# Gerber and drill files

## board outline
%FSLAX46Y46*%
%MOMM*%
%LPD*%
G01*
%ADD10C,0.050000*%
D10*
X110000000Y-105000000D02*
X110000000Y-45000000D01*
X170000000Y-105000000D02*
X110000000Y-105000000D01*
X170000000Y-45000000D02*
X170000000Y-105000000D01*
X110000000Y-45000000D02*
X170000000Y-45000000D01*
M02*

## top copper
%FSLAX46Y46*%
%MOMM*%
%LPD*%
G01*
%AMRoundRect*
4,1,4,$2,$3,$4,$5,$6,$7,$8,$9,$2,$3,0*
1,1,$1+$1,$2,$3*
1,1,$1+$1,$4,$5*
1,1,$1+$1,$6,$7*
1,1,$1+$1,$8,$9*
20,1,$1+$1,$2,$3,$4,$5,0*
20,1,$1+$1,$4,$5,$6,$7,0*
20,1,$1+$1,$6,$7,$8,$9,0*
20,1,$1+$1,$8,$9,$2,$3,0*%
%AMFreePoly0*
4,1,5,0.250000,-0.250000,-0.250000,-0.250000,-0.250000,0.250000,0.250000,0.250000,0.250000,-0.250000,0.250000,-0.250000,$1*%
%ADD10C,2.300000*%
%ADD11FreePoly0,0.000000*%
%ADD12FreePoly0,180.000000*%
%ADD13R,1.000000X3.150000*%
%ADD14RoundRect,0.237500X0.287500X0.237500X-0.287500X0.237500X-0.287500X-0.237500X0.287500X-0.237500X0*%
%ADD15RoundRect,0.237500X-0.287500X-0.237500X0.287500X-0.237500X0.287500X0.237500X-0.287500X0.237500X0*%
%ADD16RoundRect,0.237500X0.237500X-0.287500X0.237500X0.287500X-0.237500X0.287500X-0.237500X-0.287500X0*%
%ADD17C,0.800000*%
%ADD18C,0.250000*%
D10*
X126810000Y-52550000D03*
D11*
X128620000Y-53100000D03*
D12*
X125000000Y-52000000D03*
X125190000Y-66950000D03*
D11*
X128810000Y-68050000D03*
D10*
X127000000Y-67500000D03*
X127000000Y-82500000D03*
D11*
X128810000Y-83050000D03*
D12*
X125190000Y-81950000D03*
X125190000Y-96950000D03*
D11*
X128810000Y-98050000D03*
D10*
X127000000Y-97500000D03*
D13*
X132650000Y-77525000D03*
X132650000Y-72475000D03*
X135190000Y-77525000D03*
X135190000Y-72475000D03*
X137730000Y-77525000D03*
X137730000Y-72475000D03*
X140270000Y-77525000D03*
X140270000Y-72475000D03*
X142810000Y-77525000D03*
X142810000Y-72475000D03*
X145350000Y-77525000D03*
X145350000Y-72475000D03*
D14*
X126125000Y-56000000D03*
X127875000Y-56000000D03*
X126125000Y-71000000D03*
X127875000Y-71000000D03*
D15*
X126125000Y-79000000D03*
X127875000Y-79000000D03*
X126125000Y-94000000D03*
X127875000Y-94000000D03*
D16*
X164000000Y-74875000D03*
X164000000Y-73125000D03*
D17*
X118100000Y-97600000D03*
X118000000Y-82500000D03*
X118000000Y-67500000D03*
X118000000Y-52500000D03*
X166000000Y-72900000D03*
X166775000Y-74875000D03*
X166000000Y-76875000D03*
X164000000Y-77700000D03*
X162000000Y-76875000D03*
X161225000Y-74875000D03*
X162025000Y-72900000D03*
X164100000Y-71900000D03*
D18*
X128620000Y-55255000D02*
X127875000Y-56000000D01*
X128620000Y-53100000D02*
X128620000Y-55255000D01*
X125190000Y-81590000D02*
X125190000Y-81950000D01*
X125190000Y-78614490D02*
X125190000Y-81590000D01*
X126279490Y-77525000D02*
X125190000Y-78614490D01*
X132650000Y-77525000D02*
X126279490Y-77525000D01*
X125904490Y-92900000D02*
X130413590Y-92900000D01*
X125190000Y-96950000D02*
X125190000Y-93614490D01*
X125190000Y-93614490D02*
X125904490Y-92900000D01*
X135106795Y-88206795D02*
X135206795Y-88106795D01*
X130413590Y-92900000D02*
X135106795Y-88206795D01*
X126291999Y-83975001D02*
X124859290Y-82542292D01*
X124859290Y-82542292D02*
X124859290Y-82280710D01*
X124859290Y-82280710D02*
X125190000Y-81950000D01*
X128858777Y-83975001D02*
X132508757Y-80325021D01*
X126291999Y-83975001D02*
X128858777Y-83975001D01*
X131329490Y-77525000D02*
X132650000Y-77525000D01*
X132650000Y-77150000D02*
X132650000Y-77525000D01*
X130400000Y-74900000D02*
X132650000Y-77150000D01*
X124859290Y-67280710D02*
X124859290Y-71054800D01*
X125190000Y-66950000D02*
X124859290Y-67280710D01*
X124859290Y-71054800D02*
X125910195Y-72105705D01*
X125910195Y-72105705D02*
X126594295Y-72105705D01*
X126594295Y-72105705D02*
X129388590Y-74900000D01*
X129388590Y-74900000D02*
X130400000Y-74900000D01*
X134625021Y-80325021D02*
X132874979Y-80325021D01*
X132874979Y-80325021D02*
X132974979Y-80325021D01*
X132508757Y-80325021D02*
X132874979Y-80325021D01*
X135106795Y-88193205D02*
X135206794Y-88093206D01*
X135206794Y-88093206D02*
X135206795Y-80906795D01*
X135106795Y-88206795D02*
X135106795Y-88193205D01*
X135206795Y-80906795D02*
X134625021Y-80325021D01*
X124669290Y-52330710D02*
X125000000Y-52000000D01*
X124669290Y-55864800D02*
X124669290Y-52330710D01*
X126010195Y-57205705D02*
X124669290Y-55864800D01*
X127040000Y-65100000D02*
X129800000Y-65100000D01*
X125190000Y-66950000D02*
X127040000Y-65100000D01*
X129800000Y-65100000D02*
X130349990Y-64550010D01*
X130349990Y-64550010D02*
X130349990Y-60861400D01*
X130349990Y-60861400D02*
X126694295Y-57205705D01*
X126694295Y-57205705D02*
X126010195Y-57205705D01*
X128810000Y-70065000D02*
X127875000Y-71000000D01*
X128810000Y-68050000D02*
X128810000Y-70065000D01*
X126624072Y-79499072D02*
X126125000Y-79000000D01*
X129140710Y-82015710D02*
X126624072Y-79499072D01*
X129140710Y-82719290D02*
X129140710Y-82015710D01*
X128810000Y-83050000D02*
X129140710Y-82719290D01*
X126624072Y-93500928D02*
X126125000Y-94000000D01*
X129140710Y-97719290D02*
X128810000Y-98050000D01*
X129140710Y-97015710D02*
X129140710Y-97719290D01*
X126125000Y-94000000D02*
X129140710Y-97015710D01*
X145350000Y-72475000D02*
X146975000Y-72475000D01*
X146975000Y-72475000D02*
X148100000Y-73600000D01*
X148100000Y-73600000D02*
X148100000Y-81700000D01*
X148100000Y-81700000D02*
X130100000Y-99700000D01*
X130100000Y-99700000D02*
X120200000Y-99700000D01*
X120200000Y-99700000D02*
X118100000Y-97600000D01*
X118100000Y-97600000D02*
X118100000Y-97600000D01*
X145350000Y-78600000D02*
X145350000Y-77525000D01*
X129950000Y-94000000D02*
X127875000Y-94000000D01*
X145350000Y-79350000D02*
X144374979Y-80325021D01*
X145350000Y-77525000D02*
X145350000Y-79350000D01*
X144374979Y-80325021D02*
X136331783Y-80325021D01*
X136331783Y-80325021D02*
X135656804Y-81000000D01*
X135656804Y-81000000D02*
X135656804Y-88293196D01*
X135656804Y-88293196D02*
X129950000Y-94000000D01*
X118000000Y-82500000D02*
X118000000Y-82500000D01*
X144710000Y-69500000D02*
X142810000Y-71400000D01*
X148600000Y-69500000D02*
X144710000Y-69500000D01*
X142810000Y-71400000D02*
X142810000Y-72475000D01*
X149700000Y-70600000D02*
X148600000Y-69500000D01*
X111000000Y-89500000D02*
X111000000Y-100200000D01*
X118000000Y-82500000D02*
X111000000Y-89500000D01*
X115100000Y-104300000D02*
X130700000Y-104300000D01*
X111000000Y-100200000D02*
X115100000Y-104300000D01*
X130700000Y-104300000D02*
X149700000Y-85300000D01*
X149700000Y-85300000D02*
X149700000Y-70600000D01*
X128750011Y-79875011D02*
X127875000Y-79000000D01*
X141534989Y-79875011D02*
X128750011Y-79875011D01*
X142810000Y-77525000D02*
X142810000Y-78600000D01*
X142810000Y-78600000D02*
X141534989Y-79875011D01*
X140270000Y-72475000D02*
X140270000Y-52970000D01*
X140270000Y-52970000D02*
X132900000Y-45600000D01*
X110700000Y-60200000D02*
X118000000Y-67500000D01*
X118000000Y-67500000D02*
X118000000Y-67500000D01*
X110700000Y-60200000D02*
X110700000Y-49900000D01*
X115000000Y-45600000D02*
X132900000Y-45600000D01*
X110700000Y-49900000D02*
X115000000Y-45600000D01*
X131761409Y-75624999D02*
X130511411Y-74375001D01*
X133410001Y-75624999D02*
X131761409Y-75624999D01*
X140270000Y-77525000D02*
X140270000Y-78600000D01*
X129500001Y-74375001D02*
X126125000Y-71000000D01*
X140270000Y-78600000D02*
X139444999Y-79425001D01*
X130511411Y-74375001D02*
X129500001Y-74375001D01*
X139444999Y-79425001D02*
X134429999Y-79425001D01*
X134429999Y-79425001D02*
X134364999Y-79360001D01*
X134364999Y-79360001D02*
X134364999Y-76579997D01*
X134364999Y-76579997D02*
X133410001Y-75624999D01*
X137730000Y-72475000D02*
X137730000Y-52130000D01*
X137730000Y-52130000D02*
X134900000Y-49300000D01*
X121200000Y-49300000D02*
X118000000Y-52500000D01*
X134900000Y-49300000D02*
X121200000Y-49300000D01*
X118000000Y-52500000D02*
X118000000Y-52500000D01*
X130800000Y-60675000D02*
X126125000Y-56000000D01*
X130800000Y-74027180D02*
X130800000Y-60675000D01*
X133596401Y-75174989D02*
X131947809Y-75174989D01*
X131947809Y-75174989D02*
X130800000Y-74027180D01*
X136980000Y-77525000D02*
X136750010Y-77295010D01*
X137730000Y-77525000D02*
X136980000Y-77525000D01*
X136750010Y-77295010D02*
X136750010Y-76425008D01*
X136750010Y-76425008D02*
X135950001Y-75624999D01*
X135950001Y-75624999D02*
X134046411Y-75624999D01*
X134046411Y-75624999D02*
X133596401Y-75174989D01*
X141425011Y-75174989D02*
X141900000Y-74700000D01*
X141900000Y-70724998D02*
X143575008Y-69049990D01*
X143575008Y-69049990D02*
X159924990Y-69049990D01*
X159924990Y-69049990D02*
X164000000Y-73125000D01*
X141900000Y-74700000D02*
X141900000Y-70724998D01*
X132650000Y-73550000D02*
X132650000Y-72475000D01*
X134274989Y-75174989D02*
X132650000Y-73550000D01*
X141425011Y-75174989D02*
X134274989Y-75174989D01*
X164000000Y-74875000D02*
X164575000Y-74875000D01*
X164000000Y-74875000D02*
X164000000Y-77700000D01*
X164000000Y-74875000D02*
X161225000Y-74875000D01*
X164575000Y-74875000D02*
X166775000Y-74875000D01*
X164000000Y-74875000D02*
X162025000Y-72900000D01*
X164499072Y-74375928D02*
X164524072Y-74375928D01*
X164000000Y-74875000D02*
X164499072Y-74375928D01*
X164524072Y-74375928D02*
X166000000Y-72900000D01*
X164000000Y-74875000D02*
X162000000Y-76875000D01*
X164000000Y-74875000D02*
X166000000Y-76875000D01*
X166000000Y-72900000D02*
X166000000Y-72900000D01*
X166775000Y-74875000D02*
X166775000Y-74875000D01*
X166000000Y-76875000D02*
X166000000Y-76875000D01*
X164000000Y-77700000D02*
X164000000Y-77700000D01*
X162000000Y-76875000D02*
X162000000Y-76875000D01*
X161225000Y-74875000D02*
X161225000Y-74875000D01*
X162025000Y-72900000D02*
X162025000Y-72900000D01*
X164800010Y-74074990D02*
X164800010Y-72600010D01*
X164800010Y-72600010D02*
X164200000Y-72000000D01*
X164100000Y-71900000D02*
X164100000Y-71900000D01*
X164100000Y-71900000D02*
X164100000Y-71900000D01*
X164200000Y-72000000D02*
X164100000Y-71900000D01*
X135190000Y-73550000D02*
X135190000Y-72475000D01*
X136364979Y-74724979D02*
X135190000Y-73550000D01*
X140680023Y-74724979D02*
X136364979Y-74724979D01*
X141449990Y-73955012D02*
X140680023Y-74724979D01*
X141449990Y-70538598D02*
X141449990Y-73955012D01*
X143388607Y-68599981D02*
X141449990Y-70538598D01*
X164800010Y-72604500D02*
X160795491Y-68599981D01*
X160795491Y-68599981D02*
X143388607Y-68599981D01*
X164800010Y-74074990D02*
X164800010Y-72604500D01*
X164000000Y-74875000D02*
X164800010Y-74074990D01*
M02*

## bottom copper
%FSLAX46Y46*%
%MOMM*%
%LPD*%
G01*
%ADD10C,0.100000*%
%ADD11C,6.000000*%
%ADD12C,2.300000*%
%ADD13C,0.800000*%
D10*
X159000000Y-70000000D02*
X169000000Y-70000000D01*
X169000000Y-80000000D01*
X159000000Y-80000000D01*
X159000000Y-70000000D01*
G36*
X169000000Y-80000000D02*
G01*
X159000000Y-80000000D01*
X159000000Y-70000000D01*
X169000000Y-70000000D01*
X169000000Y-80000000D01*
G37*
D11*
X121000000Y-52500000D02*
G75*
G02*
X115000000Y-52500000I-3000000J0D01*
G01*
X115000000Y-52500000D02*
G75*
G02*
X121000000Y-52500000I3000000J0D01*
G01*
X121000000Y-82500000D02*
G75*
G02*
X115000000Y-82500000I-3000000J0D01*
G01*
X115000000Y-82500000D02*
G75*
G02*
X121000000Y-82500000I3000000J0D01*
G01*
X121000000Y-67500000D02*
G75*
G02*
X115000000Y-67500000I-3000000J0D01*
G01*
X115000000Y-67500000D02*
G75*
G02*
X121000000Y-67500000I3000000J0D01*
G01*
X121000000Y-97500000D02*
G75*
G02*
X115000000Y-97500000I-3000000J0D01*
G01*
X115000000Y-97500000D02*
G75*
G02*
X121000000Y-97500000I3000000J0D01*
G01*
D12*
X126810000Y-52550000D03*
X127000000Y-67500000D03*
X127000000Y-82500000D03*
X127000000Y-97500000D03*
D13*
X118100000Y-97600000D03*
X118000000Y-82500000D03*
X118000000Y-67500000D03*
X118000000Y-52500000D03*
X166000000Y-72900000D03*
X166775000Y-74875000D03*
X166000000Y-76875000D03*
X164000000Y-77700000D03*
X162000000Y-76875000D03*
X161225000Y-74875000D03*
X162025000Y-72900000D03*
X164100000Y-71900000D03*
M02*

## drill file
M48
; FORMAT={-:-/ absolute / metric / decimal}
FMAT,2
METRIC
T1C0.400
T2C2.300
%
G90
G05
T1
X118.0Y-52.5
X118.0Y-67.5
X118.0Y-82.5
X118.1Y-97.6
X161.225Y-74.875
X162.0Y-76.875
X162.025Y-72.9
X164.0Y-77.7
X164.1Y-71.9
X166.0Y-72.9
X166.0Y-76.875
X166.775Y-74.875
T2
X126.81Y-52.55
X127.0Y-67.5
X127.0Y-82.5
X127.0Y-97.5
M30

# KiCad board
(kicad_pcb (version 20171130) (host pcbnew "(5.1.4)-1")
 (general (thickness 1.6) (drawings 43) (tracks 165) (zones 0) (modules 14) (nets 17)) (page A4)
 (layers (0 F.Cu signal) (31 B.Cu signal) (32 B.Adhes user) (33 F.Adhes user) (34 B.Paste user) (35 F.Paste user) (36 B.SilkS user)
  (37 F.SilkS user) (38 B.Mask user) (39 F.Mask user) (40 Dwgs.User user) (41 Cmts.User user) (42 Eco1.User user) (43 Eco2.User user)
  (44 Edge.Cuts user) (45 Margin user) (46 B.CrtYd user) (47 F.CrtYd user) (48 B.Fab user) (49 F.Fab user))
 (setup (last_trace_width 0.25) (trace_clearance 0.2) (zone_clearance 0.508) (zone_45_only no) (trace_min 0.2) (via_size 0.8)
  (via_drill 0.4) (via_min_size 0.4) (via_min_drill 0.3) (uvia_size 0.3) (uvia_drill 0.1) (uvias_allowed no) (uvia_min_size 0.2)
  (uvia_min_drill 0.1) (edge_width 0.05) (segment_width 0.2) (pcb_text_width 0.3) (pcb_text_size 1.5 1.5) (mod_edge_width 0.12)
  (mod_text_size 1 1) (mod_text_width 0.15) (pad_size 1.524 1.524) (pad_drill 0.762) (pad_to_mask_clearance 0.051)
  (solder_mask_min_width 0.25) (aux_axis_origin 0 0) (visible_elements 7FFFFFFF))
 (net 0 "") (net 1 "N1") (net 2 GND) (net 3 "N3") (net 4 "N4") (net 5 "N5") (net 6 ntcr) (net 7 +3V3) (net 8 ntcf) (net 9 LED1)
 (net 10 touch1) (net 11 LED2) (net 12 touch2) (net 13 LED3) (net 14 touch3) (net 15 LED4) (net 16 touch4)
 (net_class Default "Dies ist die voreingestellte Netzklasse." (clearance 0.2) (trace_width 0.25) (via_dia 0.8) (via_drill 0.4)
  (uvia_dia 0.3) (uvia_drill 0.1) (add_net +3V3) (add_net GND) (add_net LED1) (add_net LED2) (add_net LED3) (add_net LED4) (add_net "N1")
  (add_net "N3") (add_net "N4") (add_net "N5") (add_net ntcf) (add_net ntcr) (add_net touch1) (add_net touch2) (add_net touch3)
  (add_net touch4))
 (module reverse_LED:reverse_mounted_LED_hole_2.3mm (layer F.Cu) (at 126.81 52.55)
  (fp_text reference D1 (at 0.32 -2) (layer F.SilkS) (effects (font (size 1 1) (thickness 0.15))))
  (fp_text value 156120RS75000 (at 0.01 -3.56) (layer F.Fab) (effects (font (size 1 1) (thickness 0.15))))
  (pad 0 thru_hole circle (at 0 0) (size 2.3 2.3) (drill 2.3) (layers *.Cu *.Mask))
  (pad 2 smd custom (at 1.81 0.55) (size 0.5 0.5) (layers F.Cu F.Paste F.Mask) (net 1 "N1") (zone_connect 0)
   (options (clearance outline) (anchor rect)) (primitives))
  (pad 1 smd custom (at -1.81 -0.55 180) (size 0.5 0.5) (layers F.Cu F.Paste F.Mask) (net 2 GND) (zone_connect 0)
   (options (clearance outline) (anchor rect)) (primitives)))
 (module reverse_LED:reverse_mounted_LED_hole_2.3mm (layer F.Cu) (at 127 67.5)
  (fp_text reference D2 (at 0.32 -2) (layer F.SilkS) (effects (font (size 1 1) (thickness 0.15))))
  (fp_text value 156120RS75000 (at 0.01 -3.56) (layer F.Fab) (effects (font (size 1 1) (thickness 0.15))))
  (pad 1 smd custom (at -1.81 -0.55 180) (size 0.5 0.5) (layers F.Cu F.Paste F.Mask) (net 2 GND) (zone_connect 0)
   (options (clearance outline) (anchor rect)) (primitives))
  (pad 2 smd custom (at 1.81 0.55) (size 0.5 0.5) (layers F.Cu F.Paste F.Mask) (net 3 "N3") (zone_connect 0)
   (options (clearance outline) (anchor rect)) (primitives))
  (pad 0 thru_hole circle (at 0 0) (size 2.3 2.3) (drill 2.3) (layers *.Cu *.Mask)))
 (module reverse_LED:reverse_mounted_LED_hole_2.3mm (layer F.Cu) (at 127 82.5)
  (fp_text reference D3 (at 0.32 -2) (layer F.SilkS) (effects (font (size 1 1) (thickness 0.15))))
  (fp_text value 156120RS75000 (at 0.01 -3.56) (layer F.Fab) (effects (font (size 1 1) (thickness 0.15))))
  (pad 0 thru_hole circle (at 0 0) (size 2.3 2.3) (drill 2.3) (layers *.Cu *.Mask))
  (pad 2 smd custom (at 1.81 0.55) (size 0.5 0.5) (layers F.Cu F.Paste F.Mask) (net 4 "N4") (zone_connect 0)
   (options (clearance outline) (anchor rect)) (primitives))
  (pad 1 smd custom (at -1.81 -0.55 180) (size 0.5 0.5) (layers F.Cu F.Paste F.Mask) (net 2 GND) (zone_connect 0)
   (options (clearance outline) (anchor rect)) (primitives)))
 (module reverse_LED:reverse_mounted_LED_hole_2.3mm (layer F.Cu) (at 127 97.5)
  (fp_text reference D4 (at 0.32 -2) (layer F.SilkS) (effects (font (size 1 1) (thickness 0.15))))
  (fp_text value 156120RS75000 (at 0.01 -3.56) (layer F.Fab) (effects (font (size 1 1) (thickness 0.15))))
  (pad 1 smd custom (at -1.81 -0.55 180) (size 0.5 0.5) (layers F.Cu F.Paste F.Mask) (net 2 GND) (zone_connect 0)
   (options (clearance outline) (anchor rect)) (primitives))
  (pad 2 smd custom (at 1.81 0.55) (size 0.5 0.5) (layers F.Cu F.Paste F.Mask) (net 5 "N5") (zone_connect 0)
   (options (clearance outline) (anchor rect)) (primitives))
  (pad 0 thru_hole circle (at 0 0) (size 2.3 2.3) (drill 2.3) (layers *.Cu *.Mask)))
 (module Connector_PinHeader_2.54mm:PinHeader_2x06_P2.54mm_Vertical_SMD (layer F.Cu) (at 139 75 90)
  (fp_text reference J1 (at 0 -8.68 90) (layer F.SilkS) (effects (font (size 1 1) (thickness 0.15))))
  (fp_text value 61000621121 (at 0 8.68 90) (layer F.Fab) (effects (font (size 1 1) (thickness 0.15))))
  (pad 1 smd rect (at -2.525 -6.35 90) (size 3.15 1) (layers F.Cu F.Paste F.Mask) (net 2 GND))
  (pad 2 smd rect (at 2.525 -6.35 90) (size 3.15 1) (layers F.Cu F.Paste F.Mask) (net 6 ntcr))
  (pad 3 smd rect (at -2.525 -3.81 90) (size 3.15 1) (layers F.Cu F.Paste F.Mask) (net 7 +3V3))
  (pad 4 smd rect (at 2.525 -3.81 90) (size 3.15 1) (layers F.Cu F.Paste F.Mask) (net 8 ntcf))
  (pad 5 smd rect (at -2.525 -1.27 90) (size 3.15 1) (layers F.Cu F.Paste F.Mask) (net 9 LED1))
  (pad 6 smd rect (at 2.525 -1.27 90) (size 3.15 1) (layers F.Cu F.Paste F.Mask) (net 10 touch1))
  (pad 7 smd rect (at -2.525 1.27 90) (size 3.15 1) (layers F.Cu F.Paste F.Mask) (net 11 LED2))
  (pad 8 smd rect (at 2.525 1.27 90) (size 3.15 1) (layers F.Cu F.Paste F.Mask) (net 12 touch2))
  (pad 9 smd rect (at -2.525 3.81 90) (size 3.15 1) (layers F.Cu F.Paste F.Mask) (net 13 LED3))
  (pad 10 smd rect (at 2.525 3.81 90) (size 3.15 1) (layers F.Cu F.Paste F.Mask) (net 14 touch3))
  (pad 11 smd rect (at -2.525 6.35 90) (size 3.15 1) (layers F.Cu F.Paste F.Mask) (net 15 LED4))
  (pad 12 smd rect (at 2.525 6.35 90) (size 3.15 1) (layers F.Cu F.Paste F.Mask) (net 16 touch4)))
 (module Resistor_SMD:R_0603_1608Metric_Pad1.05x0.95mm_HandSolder (layer F.Cu) (at 127 56 180)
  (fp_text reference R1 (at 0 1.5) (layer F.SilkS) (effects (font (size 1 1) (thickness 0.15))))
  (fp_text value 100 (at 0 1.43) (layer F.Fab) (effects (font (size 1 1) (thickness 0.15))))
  (pad 2 smd roundrect (at 0.875 0 180) (size 1.05 0.95) (layers F.Cu F.Paste F.Mask) (roundrect_rratio 0.25) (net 9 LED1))
  (pad 1 smd roundrect (at -0.875 0 180) (size 1.05 0.95) (layers F.Cu F.Paste F.Mask) (roundrect_rratio 0.25) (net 1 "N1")))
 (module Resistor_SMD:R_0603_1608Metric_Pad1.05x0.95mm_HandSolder (layer F.Cu) (at 127 71 180)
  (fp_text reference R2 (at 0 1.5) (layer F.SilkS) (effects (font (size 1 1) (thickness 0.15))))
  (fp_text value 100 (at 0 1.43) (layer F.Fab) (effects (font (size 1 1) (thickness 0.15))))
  (pad 2 smd roundrect (at 0.875 0 180) (size 1.05 0.95) (layers F.Cu F.Paste F.Mask) (roundrect_rratio 0.25) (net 11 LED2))
  (pad 1 smd roundrect (at -0.875 0 180) (size 1.05 0.95) (layers F.Cu F.Paste F.Mask) (roundrect_rratio 0.25) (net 3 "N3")))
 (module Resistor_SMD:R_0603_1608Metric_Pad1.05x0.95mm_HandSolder (layer F.Cu) (at 127 79)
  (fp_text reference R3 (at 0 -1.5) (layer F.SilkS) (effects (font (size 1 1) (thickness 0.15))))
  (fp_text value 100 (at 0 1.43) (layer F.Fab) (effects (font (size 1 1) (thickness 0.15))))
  (pad 1 smd roundrect (at -0.875 0) (size 1.05 0.95) (layers F.Cu F.Paste F.Mask) (roundrect_rratio 0.25) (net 4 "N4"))
  (pad 2 smd roundrect (at 0.875 0) (size 1.05 0.95) (layers F.Cu F.Paste F.Mask) (roundrect_rratio 0.25) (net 13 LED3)))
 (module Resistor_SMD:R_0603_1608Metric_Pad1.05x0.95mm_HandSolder (layer F.Cu) (at 127 94)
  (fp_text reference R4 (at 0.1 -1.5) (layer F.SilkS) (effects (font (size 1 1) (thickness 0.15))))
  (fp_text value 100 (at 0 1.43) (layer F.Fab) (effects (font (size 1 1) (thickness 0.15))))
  (pad 1 smd roundrect (at -0.875 0) (size 1.05 0.95) (layers F.Cu F.Paste F.Mask) (roundrect_rratio 0.25) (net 5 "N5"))
  (pad 2 smd roundrect (at 0.875 0) (size 1.05 0.95) (layers F.Cu F.Paste F.Mask) (roundrect_rratio 0.25) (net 15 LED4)))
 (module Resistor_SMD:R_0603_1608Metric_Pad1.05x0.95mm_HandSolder (layer F.Cu) (at 164 74 90)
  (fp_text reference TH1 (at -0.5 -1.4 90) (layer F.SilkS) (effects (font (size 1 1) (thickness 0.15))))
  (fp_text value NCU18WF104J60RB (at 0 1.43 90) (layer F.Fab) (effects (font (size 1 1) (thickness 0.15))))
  (pad 1 smd roundrect (at -0.875 0 90) (size 1.05 0.95) (layers F.Cu F.Paste F.Mask) (roundrect_rratio 0.25) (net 8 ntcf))
  (pad 2 smd roundrect (at 0.875 0 90) (size 1.05 0.95) (layers F.Cu F.Paste F.Mask) (roundrect_rratio 0.25) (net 6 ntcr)))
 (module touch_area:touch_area (layer F.Cu) (at 118 52.5)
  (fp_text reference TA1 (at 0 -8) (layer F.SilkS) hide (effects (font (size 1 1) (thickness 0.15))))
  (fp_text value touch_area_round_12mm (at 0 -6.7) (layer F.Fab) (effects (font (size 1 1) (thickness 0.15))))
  (fp_circle (center 0 0) (end 3 0) (layer B.Cu) (width 6)))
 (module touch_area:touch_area (layer F.Cu) (at 118 82.5)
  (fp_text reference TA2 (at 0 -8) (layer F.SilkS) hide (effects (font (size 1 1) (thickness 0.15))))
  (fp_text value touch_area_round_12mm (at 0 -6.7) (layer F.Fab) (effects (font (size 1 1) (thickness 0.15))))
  (fp_circle (center 0 0) (end 3 0) (layer B.Cu) (width 6)))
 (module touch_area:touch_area (layer F.Cu) (at 118 67.5)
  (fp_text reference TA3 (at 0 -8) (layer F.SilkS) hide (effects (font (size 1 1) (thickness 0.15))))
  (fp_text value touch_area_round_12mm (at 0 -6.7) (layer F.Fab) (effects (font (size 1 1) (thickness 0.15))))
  (fp_circle (center 0 0) (end 3 0) (layer B.Cu) (width 6)))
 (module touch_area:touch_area (layer F.Cu) (at 118 97.5)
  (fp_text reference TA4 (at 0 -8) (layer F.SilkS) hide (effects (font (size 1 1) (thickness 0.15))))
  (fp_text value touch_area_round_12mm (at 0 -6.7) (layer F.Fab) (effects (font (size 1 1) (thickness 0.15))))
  (fp_circle (center 0 0) (end 3 0) (layer B.Cu) (width 6)))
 (gr_poly (pts (xy 159 70) (xy 169 70) (xy 169 80) (xy 159 80)) (layer B.Cu) (width 0.1))
 (gr_line (start 110 105) (end 110 45) (layer Edge.Cuts) (width 0.05))
 (gr_line (start 170 105) (end 110 105) (layer Edge.Cuts) (width 0.05))
 (gr_line (start 170 45) (end 170 105) (layer Edge.Cuts) (width 0.05))
 (gr_line (start 110 45) (end 170 45) (layer Edge.Cuts) (width 0.05))
 (segment (start 128.62 55.255) (end 127.875 56) (width 0.25) (layer F.Cu) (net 1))
 (segment (start 128.62 53.1) (end 128.62 55.255) (width 0.25) (layer F.Cu) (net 1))
 (segment (start 125.19 81.59) (end 125.19 81.95) (width 0.25) (layer F.Cu) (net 2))
 (segment (start 125.19 78.61449) (end 125.19 81.59) (width 0.25) (layer F.Cu) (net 2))
 (segment (start 126.27949 77.525) (end 125.19 78.61449) (width 0.25) (layer F.Cu) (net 2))
 (segment (start 132.65 77.525) (end 126.27949 77.525) (width 0.25) (layer F.Cu) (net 2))
 (segment (start 125.90449 92.9) (end 130.41359 92.9) (width 0.25) (layer F.Cu) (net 2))
 (segment (start 125.19 96.95) (end 125.19 93.61449) (width 0.25) (layer F.Cu) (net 2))
 (segment (start 125.19 93.61449) (end 125.90449 92.9) (width 0.25) (layer F.Cu) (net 2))
 (segment (start 135.106795 88.206795) (end 135.206795 88.106795) (width 0.25) (layer F.Cu) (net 2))
 (segment (start 130.41359 92.9) (end 135.106795 88.206795) (width 0.25) (layer F.Cu) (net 2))
 (segment (start 126.291999 83.975001) (end 124.85929 82.542292) (width 0.25) (layer F.Cu) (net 2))
 (segment (start 124.85929 82.542292) (end 124.85929 82.28071) (width 0.25) (layer F.Cu) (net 2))
 (segment (start 124.85929 82.28071) (end 125.19 81.95) (width 0.25) (layer F.Cu) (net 2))
 (segment (start 128.858777 83.975001) (end 132.508757 80.325021) (width 0.25) (layer F.Cu) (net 2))
 (segment (start 126.291999 83.975001) (end 128.858777 83.975001) (width 0.25) (layer F.Cu) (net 2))
 (segment (start 131.32949 77.525) (end 132.65 77.525) (width 0.25) (layer F.Cu) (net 2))
 (segment (start 132.65 77.15) (end 132.65 77.525) (width 0.25) (layer F.Cu) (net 2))
 (segment (start 130.4 74.9) (end 132.65 77.15) (width 0.25) (layer F.Cu) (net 2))
 (segment (start 124.85929 67.28071) (end 124.85929 71.0548) (width 0.25) (layer F.Cu) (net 2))
 (segment (start 125.19 66.95) (end 124.85929 67.28071) (width 0.25) (layer F.Cu) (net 2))
 (segment (start 124.85929 71.0548) (end 125.910195 72.105705) (width 0.25) (layer F.Cu) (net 2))
 (segment (start 125.910195 72.105705) (end 126.594295 72.105705) (width 0.25) (layer F.Cu) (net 2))
 (segment (start 126.594295 72.105705) (end 129.38859 74.9) (width 0.25) (layer F.Cu) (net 2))
 (segment (start 129.38859 74.9) (end 130.4 74.9) (width 0.25) (layer F.Cu) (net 2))
 (segment (start 134.625021 80.325021) (end 132.874979 80.325021) (width 0.25) (layer F.Cu) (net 2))
 (segment (start 132.874979 80.325021) (end 132.974979 80.325021) (width 0.25) (layer F.Cu) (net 2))
 (segment (start 132.508757 80.325021) (end 132.874979 80.325021) (width 0.25) (layer F.Cu) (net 2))
 (segment (start 135.106795 88.193205) (end 135.206794 88.093206) (width 0.25) (layer F.Cu) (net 2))
 (segment (start 135.206794 88.093206) (end 135.206795 80.906795) (width 0.25) (layer F.Cu) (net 2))
 (segment (start 135.106795 88.206795) (end 135.106795 88.193205) (width 0.25) (layer F.Cu) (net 2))
 (segment (start 135.206795 80.906795) (end 134.625021 80.325021) (width 0.25) (layer F.Cu) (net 2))
 (segment (start 124.66929 52.33071) (end 125 52) (width 0.25) (layer F.Cu) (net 2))
 (segment (start 124.66929 55.8648) (end 124.66929 52.33071) (width 0.25) (layer F.Cu) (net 2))
 (segment (start 126.010195 57.205705) (end 124.66929 55.8648) (width 0.25) (layer F.Cu) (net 2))
 (segment (start 127.04 65.1) (end 129.8 65.1) (width 0.25) (layer F.Cu) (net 2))
 (segment (start 125.19 66.95) (end 127.04 65.1) (width 0.25) (layer F.Cu) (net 2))
 (segment (start 129.8 65.1) (end 130.34999 64.55001) (width 0.25) (layer F.Cu) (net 2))
 (segment (start 130.34999 64.55001) (end 130.34999 60.8614) (width 0.25) (layer F.Cu) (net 2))
 (segment (start 130.34999 60.8614) (end 126.694295 57.205705) (width 0.25) (layer F.Cu) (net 2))
 (segment (start 126.694295 57.205705) (end 126.010195 57.205705) (width 0.25) (layer F.Cu) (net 2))
 (segment (start 128.81 70.065) (end 127.875 71) (width 0.25) (layer F.Cu) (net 3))
 (segment (start 128.81 68.05) (end 128.81 70.065) (width 0.25) (layer F.Cu) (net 3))
 (segment (start 126.624072 79.499072) (end 126.125 79) (width 0.25) (layer F.Cu) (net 4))
 (segment (start 129.14071 82.01571) (end 126.624072 79.499072) (width 0.25) (layer F.Cu) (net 4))
 (segment (start 129.14071 82.71929) (end 129.14071 82.01571) (width 0.25) (layer F.Cu) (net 4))
 (segment (start 128.81 83.05) (end 129.14071 82.71929) (width 0.25) (layer F.Cu) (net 4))
 (segment (start 126.624072 93.500928) (end 126.125 94) (width 0.25) (layer F.Cu) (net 5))
 (segment (start 129.14071 97.71929) (end 128.81 98.05) (width 0.25) (layer F.Cu) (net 5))
 (segment (start 129.14071 97.01571) (end 129.14071 97.71929) (width 0.25) (layer F.Cu) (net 5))
 (segment (start 126.125 94) (end 129.14071 97.01571) (width 0.25) (layer F.Cu) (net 5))
 (segment (start 145.35 72.475) (end 146.975 72.475) (width 0.25) (layer F.Cu) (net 16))
 (segment (start 146.975 72.475) (end 148.1 73.6) (width 0.25) (layer F.Cu) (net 16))
 (segment (start 148.1 73.6) (end 148.1 81.7) (width 0.25) (layer F.Cu) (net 16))
 (segment (start 148.1 81.7) (end 130.1 99.7) (width 0.25) (layer F.Cu) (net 16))
 (segment (start 130.1 99.7) (end 120.2 99.7) (width 0.25) (layer F.Cu) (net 16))
 (segment (start 120.2 99.7) (end 118.1 97.6) (width 0.25) (layer F.Cu) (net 16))
 (segment (start 118.1 97.6) (end 118.1 97.6) (width 0.25) (layer F.Cu) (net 16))
 (via (at 118.1 97.6) (size 0.8) (drill 0.4) (layers F.Cu B.Cu) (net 16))
 (segment (start 145.35 78.6) (end 145.35 77.525) (width 0.25) (layer F.Cu) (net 15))
 (segment (start 129.95 94) (end 127.875 94) (width 0.25) (layer F.Cu) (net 15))
 (segment (start 145.35 79.35) (end 144.374979 80.325021) (width 0.25) (layer F.Cu) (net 15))
 (segment (start 145.35 77.525) (end 145.35 79.35) (width 0.25) (layer F.Cu) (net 15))
 (segment (start 144.374979 80.325021) (end 136.331783 80.325021) (width 0.25) (layer F.Cu) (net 15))
 (segment (start 136.331783 80.325021) (end 135.656804 81) (width 0.25) (layer F.Cu) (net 15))
 (segment (start 135.656804 81) (end 135.656804 88.293196) (width 0.25) (layer F.Cu) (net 15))
 (segment (start 135.656804 88.293196) (end 129.95 94) (width 0.25) (layer F.Cu) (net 15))
 (segment (start 118 82.5) (end 118 82.5) (width 0.25) (layer F.Cu) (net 14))
 (via (at 118 82.5) (size 0.8) (drill 0.4) (layers F.Cu B.Cu) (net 14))
 (segment (start 144.71 69.5) (end 142.81 71.4) (width 0.25) (layer F.Cu) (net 14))
 (segment (start 148.6 69.5) (end 144.71 69.5) (width 0.25) (layer F.Cu) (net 14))
 (segment (start 142.81 71.4) (end 142.81 72.475) (width 0.25) (layer F.Cu) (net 14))
 (segment (start 149.7 70.6) (end 148.6 69.5) (width 0.25) (layer F.Cu) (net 14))
 (segment (start 111 89.5) (end 111 100.2) (width 0.25) (layer F.Cu) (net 14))
 (segment (start 118 82.5) (end 111 89.5) (width 0.25) (layer F.Cu) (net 14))
 (segment (start 115.1 104.3) (end 130.7 104.3) (width 0.25) (layer F.Cu) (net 14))
 (segment (start 111 100.2) (end 115.1 104.3) (width 0.25) (layer F.Cu) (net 14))
 (segment (start 130.7 104.3) (end 149.7 85.3) (width 0.25) (layer F.Cu) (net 14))
 (segment (start 149.7 85.3) (end 149.7 70.6) (width 0.25) (layer F.Cu) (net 14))
 (segment (start 128.750011 79.875011) (end 127.875 79) (width 0.25) (layer F.Cu) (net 13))
 (segment (start 141.534989 79.875011) (end 128.750011 79.875011) (width 0.25) (layer F.Cu) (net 13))
 (segment (start 142.81 77.525) (end 142.81 78.6) (width 0.25) (layer F.Cu) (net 13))
 (segment (start 142.81 78.6) (end 141.534989 79.875011) (width 0.25) (layer F.Cu) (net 13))
 (segment (start 140.27 72.475) (end 140.27 52.97) (width 0.25) (layer F.Cu) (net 12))
 (segment (start 140.27 52.97) (end 132.9 45.6) (width 0.25) (layer F.Cu) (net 12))
 (segment (start 110.7 60.2) (end 118 67.5) (width 0.25) (layer F.Cu) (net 12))
 (segment (start 118 67.5) (end 118 67.5) (width 0.25) (layer F.Cu) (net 12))
 (via (at 118 67.5) (size 0.8) (drill 0.4) (layers F.Cu B.Cu) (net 12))
 (segment (start 110.7 60.2) (end 110.7 49.9) (width 0.25) (layer F.Cu) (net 12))
 (segment (start 115 45.6) (end 132.9 45.6) (width 0.25) (layer F.Cu) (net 12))
 (segment (start 110.7 49.9) (end 115 45.6) (width 0.25) (layer F.Cu) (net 12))
 (segment (start 131.761409 75.624999) (end 130.511411 74.375001) (width 0.25) (layer F.Cu) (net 11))
 (segment (start 133.410001 75.624999) (end 131.761409 75.624999) (width 0.25) (layer F.Cu) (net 11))
 (segment (start 140.27 77.525) (end 140.27 78.6) (width 0.25) (layer F.Cu) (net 11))
 (segment (start 129.500001 74.375001) (end 126.125 71) (width 0.25) (layer F.Cu) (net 11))
 (segment (start 140.27 78.6) (end 139.444999 79.425001) (width 0.25) (layer F.Cu) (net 11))
 (segment (start 130.511411 74.375001) (end 129.500001 74.375001) (width 0.25) (layer F.Cu) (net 11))
 (segment (start 139.444999 79.425001) (end 134.429999 79.425001) (width 0.25) (layer F.Cu) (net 11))
 (segment (start 134.429999 79.425001) (end 134.364999 79.360001) (width 0.25) (layer F.Cu) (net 11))
 (segment (start 134.364999 79.360001) (end 134.364999 76.579997) (width 0.25) (layer F.Cu) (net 11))
 (segment (start 134.364999 76.579997) (end 133.410001 75.624999) (width 0.25) (layer F.Cu) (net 11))
 (segment (start 137.73 72.475) (end 137.73 52.13) (width 0.25) (layer F.Cu) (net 10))
 (segment (start 137.73 52.13) (end 134.9 49.3) (width 0.25) (layer F.Cu) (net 10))
 (segment (start 121.2 49.3) (end 118 52.5) (width 0.25) (layer F.Cu) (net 10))
 (segment (start 134.9 49.3) (end 121.2 49.3) (width 0.25) (layer F.Cu) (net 10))
 (segment (start 118 52.5) (end 118 52.5) (width 0.25) (layer F.Cu) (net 10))
 (via (at 118 52.5) (size 0.8) (drill 0.4) (layers F.Cu B.Cu) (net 10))
 (segment (start 130.8 60.675) (end 126.125 56) (width 0.25) (layer F.Cu) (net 9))
 (segment (start 130.8 74.02718) (end 130.8 60.675) (width 0.25) (layer F.Cu) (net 9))
 (segment (start 133.596401 75.174989) (end 131.947809 75.174989) (width 0.25) (layer F.Cu) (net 9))
 (segment (start 131.947809 75.174989) (end 130.8 74.02718) (width 0.25) (layer F.Cu) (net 9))
 (segment (start 136.98 77.525) (end 136.75001 77.29501) (width 0.25) (layer F.Cu) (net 9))
 (segment (start 137.73 77.525) (end 136.98 77.525) (width 0.25) (layer F.Cu) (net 9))
 (segment (start 136.75001 77.29501) (end 136.75001 76.425008) (width 0.25) (layer F.Cu) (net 9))
 (segment (start 136.75001 76.425008) (end 135.950001 75.624999) (width 0.25) (layer F.Cu) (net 9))
 (segment (start 135.950001 75.624999) (end 134.046411 75.624999) (width 0.25) (layer F.Cu) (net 9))
 (segment (start 134.046411 75.624999) (end 133.596401 75.174989) (width 0.25) (layer F.Cu) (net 9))
 (segment (start 141.425011 75.174989) (end 141.9 74.7) (width 0.25) (layer F.Cu) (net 6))
 (segment (start 141.9 70.724998) (end 143.575008 69.04999) (width 0.25) (layer F.Cu) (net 6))
 (segment (start 143.575008 69.04999) (end 159.92499 69.04999) (width 0.25) (layer F.Cu) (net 6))
 (segment (start 159.92499 69.04999) (end 164 73.125) (width 0.25) (layer F.Cu) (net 6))
 (segment (start 141.9 74.7) (end 141.9 70.724998) (width 0.25) (layer F.Cu) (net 6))
 (segment (start 132.65 73.55) (end 132.65 72.475) (width 0.25) (layer F.Cu) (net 6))
 (segment (start 134.274989 75.174989) (end 132.65 73.55) (width 0.25) (layer F.Cu) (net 6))
 (segment (start 141.425011 75.174989) (end 134.274989 75.174989) (width 0.25) (layer F.Cu) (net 6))
 (segment (start 164 74.875) (end 164.575 74.875) (width 0.25) (layer F.Cu) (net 8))
 (segment (start 164 74.875) (end 164 77.7) (width 0.25) (layer F.Cu) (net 8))
 (segment (start 164 74.875) (end 161.225 74.875) (width 0.25) (layer F.Cu) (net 8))
 (segment (start 164.575 74.875) (end 166.775 74.875) (width 0.25) (layer F.Cu) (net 8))
 (segment (start 164 74.875) (end 162.025 72.9) (width 0.25) (layer F.Cu) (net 8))
 (segment (start 164.499072 74.375928) (end 164.524072 74.375928) (width 0.25) (layer F.Cu) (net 8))
 (segment (start 164 74.875) (end 164.499072 74.375928) (width 0.25) (layer F.Cu) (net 8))
 (segment (start 164.524072 74.375928) (end 166 72.9) (width 0.25) (layer F.Cu) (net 8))
 (segment (start 164 74.875) (end 162 76.875) (width 0.25) (layer F.Cu) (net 8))
 (segment (start 164 74.875) (end 166 76.875) (width 0.25) (layer F.Cu) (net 8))
 (segment (start 166 72.9) (end 166 72.9) (width 0.25) (layer F.Cu) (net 8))
 (via (at 166 72.9) (size 0.8) (drill 0.4) (layers F.Cu B.Cu) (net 8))
 (segment (start 166.775 74.875) (end 166.775 74.875) (width 0.25) (layer F.Cu) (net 8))
 (via (at 166.775 74.875) (size 0.8) (drill 0.4) (layers F.Cu B.Cu) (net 8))
 (segment (start 166 76.875) (end 166 76.875) (width 0.25) (layer F.Cu) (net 8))
 (via (at 166 76.875) (size 0.8) (drill 0.4) (layers F.Cu B.Cu) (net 8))
 (segment (start 164 77.7) (end 164 77.7) (width 0.25) (layer F.Cu) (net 8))
 (via (at 164 77.7) (size 0.8) (drill 0.4) (layers F.Cu B.Cu) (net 8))
 (segment (start 162 76.875) (end 162 76.875) (width 0.25) (layer F.Cu) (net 8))
 (via (at 162 76.875) (size 0.8) (drill 0.4) (layers F.Cu B.Cu) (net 8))
 (segment (start 161.225 74.875) (end 161.225 74.875) (width 0.25) (layer F.Cu) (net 8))
 (via (at 161.225 74.875) (size 0.8) (drill 0.4) (layers F.Cu B.Cu) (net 8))
 (segment (start 162.025 72.9) (end 162.025 72.9) (width 0.25) (layer F.Cu) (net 8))
 (via (at 162.025 72.9) (size 0.8) (drill 0.4) (layers F.Cu B.Cu) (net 8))
 (segment (start 164.80001 74.07499) (end 164.80001 72.60001) (width 0.25) (layer F.Cu) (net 8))
 (segment (start 164.80001 72.60001) (end 164.2 72) (width 0.25) (layer F.Cu) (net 8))
 (segment (start 164.1 71.9) (end 164.1 71.9) (width 0.25) (layer F.Cu) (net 8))
 (segment (start 164.1 71.9) (end 164.1 71.9) (width 0.25) (layer F.Cu) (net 8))
 (segment (start 164.2 72) (end 164.1 71.9) (width 0.25) (layer F.Cu) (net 8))
 (via (at 164.1 71.9) (size 0.8) (drill 0.4) (layers F.Cu B.Cu) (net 8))
 (segment (start 135.19 73.55) (end 135.19 72.475) (width 0.25) (layer F.Cu) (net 8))
 (segment (start 136.364979 74.724979) (end 135.19 73.55) (width 0.25) (layer F.Cu) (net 8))
 (segment (start 140.680023 74.724979) (end 136.364979 74.724979) (width 0.25) (layer F.Cu) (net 8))
 (segment (start 141.44999 73.955012) (end 140.680023 74.724979) (width 0.25) (layer F.Cu) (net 8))
 (segment (start 141.44999 70.538598) (end 141.44999 73.955012) (width 0.25) (layer F.Cu) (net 8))
 (segment (start 143.388607 68.599981) (end 141.44999 70.538598) (width 0.25) (layer F.Cu) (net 8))
 (segment (start 164.80001 72.6045) (end 160.795491 68.599981) (width 0.25) (layer F.Cu) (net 8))
 (segment (start 160.795491 68.599981) (end 143.388607 68.599981) (width 0.25) (layer F.Cu) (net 8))
 (segment (start 164.80001 74.07499) (end 164.80001 72.6045) (width 0.25) (layer F.Cu) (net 8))
 (segment (start 164 74.875) (end 164.80001 74.07499) (width 0.25) (layer F.Cu) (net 8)))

